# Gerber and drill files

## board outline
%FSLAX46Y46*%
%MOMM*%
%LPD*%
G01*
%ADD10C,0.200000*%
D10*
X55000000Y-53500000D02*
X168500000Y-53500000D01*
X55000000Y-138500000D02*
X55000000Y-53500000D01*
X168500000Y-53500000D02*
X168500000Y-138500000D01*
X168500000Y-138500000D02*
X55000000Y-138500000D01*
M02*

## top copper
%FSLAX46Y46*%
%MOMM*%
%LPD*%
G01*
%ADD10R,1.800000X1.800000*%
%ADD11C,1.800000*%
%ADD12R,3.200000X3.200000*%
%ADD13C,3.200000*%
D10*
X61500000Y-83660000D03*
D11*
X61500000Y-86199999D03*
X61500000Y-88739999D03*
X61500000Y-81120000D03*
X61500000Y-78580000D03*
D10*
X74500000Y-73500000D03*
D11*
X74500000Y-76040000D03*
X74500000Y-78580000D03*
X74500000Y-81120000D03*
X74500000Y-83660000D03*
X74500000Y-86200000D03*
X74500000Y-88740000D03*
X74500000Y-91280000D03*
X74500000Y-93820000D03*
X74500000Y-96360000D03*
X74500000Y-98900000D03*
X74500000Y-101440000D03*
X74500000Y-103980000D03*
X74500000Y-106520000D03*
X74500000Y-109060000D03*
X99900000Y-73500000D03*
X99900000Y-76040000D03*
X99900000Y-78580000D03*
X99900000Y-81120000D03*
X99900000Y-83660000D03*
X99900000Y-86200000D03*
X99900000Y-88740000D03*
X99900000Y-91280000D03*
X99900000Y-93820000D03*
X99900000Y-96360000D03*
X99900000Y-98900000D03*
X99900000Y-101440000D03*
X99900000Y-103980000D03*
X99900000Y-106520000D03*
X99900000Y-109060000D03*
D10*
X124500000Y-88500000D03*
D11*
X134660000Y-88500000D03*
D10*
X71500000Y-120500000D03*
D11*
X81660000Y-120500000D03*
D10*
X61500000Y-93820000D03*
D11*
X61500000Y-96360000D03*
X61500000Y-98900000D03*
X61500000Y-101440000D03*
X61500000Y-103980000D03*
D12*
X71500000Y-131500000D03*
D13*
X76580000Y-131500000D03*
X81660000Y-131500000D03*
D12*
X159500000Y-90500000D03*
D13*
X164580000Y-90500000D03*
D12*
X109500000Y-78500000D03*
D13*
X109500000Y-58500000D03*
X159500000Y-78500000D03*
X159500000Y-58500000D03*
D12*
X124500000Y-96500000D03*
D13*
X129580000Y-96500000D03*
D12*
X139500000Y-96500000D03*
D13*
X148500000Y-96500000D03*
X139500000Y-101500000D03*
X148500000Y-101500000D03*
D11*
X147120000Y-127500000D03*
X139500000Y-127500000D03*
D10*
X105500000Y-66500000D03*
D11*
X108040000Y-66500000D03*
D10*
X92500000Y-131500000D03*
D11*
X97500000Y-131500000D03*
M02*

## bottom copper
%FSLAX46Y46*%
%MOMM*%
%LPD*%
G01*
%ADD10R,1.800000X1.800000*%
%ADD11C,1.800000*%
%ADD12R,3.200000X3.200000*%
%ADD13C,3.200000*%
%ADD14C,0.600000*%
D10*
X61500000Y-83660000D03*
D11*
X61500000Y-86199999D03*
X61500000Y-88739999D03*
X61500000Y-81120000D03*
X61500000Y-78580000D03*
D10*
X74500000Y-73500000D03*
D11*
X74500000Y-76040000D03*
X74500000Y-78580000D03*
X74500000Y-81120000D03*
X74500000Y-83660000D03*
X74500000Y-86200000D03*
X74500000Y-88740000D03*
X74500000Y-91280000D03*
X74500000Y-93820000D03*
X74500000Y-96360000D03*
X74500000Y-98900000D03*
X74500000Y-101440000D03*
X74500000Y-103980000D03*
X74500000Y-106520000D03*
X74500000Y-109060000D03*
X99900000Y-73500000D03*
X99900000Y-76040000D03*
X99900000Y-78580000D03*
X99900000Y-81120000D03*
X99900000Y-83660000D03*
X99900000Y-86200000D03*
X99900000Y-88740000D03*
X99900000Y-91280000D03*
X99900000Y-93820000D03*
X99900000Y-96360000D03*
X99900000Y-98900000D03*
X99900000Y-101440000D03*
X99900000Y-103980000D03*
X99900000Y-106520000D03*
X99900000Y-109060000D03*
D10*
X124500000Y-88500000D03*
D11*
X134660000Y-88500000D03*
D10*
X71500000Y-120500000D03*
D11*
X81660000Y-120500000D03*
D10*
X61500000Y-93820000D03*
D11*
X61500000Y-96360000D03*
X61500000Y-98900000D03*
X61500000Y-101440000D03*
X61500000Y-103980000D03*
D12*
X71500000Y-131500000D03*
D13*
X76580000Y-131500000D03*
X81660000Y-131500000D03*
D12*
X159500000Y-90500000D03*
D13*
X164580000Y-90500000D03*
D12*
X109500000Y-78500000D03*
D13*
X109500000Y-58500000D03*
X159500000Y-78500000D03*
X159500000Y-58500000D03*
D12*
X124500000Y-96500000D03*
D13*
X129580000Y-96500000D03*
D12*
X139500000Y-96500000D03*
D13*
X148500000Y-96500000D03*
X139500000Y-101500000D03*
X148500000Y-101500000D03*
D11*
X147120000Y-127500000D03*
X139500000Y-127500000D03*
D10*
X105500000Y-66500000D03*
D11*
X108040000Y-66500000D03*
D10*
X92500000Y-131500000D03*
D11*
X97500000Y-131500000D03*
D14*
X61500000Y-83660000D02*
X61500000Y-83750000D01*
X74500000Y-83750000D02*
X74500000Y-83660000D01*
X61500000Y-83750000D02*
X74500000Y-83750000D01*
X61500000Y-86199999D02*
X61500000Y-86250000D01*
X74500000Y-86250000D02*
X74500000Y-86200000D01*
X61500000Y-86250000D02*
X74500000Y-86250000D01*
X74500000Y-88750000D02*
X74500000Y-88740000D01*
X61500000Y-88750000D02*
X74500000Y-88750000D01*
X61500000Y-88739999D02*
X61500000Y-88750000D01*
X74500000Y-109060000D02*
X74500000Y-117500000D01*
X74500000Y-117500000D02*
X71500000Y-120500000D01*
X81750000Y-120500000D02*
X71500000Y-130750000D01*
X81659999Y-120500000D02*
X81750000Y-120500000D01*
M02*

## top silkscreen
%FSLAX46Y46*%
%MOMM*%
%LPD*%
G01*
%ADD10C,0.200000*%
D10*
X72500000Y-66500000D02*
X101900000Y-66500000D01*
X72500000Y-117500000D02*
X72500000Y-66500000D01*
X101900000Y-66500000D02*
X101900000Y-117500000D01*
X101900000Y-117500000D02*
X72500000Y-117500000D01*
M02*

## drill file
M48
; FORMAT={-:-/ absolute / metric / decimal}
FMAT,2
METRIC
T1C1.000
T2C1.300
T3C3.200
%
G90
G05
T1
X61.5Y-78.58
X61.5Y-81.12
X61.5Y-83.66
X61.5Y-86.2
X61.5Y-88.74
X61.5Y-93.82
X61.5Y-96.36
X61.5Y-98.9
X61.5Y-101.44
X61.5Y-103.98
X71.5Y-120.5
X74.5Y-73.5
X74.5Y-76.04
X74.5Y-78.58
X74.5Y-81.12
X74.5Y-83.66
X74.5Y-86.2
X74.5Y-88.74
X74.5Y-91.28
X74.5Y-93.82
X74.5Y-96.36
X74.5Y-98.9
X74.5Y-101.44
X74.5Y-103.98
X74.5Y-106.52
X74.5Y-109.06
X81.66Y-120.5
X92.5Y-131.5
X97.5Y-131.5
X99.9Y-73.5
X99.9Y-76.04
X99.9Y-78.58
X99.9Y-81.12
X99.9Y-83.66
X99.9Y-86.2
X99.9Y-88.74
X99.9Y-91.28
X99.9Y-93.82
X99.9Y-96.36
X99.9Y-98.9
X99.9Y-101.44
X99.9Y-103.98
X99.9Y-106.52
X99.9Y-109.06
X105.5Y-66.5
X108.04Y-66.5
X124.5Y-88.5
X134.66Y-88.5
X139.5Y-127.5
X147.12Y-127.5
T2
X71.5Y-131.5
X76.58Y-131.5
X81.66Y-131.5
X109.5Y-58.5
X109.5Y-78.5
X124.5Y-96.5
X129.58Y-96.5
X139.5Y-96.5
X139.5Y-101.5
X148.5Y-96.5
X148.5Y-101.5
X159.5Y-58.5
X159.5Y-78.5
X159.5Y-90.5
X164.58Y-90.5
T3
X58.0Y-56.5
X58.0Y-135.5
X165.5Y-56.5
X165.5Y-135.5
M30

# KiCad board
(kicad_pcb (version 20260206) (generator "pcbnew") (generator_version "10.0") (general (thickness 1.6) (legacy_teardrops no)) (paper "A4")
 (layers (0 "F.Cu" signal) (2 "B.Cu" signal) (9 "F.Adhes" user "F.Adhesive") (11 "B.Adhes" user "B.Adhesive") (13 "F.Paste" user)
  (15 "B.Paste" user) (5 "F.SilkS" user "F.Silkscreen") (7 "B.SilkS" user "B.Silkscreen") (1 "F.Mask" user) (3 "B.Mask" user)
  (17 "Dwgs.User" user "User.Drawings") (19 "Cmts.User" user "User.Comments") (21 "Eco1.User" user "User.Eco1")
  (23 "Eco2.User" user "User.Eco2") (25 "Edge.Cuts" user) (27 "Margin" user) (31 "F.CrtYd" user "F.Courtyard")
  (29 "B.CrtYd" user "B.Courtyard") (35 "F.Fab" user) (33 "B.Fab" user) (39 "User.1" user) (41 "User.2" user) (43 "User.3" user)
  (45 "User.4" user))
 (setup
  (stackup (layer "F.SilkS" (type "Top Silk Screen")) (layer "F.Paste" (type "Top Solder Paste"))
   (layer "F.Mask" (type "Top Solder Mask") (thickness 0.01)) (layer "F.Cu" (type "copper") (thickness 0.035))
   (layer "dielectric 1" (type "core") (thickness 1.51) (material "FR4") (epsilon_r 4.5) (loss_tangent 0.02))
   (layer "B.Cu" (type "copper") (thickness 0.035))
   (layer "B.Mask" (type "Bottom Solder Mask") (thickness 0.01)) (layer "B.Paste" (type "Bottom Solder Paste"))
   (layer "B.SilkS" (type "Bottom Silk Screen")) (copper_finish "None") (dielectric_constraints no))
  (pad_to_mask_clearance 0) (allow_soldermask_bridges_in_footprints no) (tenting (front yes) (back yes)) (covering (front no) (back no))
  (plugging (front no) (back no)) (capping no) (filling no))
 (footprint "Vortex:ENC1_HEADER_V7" (layer "F.Cu") (at 61.5 83.5 -90)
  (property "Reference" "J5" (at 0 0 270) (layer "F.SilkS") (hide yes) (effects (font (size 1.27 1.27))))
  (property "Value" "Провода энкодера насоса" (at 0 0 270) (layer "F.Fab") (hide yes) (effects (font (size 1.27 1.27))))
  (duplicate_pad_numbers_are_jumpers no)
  (pad "1" thru_hole rect (at 0.16 0 270) (size 1.8 1.8) (drill 1) (layers "*.Cu") (remove_unused_layers no) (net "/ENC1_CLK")
   (thermal_bridge_angle 45))
  (pad "2" thru_hole circle (at 2.699999 0 270) (size 1.8 1.8) (drill 1) (layers "*.Cu") (remove_unused_layers no) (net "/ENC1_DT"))
  (pad "3" thru_hole circle (at 5.239999 0 270) (size 1.8 1.8) (drill 1) (layers "*.Cu") (remove_unused_layers no) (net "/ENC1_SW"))
  (pad "4" thru_hole circle (at -2.38 0 270) (size 1.8 1.8) (drill 1) (layers "*.Cu") (remove_unused_layers no) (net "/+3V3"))
  (pad "5" thru_hole circle (at -4.92 0 270) (size 1.8 1.8) (drill 1) (layers "*.Cu") (remove_unused_layers no) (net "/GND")))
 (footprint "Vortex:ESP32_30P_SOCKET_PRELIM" (layer "F.Cu") (at 74.5 73.5)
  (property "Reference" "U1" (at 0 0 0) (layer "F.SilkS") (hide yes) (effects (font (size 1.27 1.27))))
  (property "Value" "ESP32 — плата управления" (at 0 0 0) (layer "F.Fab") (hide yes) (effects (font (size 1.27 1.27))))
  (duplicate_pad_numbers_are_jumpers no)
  (fp_line (start -2 -7) (end 27.4 -7) (stroke (width 0.2) (type default)) (layer "F.SilkS"))
  (fp_line (start -2 44) (end -2 -7) (stroke (width 0.2) (type default)) (layer "F.SilkS"))
  (fp_line (start 27.4 -7) (end 27.4 44) (stroke (width 0.2) (type default)) (layer "F.SilkS"))
  (fp_line (start 27.4 44) (end -2 44) (stroke (width 0.2) (type default)) (layer "F.SilkS"))
  (pad "1" thru_hole rect (at 0 0) (size 1.8 1.8) (drill 1) (layers "*.Cu") (remove_unused_layers no) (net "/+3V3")
   (thermal_bridge_angle 45))
  (pad "2" thru_hole circle (at 0 2.54) (size 1.8 1.8) (drill 1) (layers "*.Cu") (remove_unused_layers no) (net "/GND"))
  (pad "3" thru_hole circle (at 0 5.08) (size 1.8 1.8) (drill 1) (layers "*.Cu") (remove_unused_layers no) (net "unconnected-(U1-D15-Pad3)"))
  (pad "4" thru_hole circle (at 0 7.62) (size 1.8 1.8) (drill 1) (layers "*.Cu") (remove_unused_layers no) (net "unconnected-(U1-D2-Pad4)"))
  (pad "5" thru_hole circle (at 0 10.16) (size 1.8 1.8) (drill 1) (layers "*.Cu") (remove_unused_layers no) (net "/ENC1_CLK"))
  (pad "6" thru_hole circle (at 0 12.7) (size 1.8 1.8) (drill 1) (layers "*.Cu") (remove_unused_layers no) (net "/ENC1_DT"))
  (pad "7" thru_hole circle (at 0 15.24) (size 1.8 1.8) (drill 1) (layers "*.Cu") (remove_unused_layers no) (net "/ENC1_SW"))
  (pad "8" thru_hole circle (at 0 17.78) (size 1.8 1.8) (drill 1) (layers "*.Cu") (remove_unused_layers no) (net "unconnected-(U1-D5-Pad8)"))
  (pad "9" thru_hole circle (at 0 20.32) (size 1.8 1.8) (drill 1) (layers "*.Cu") (remove_unused_layers no) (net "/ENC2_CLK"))
  (pad "10" thru_hole circle (at 0 22.86) (size 1.8 1.8) (drill 1) (layers "*.Cu") (remove_unused_layers no) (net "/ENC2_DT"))
  (pad "11" thru_hole circle (at 0 25.4) (size 1.8 1.8) (drill 1) (layers "*.Cu") (remove_unused_layers no) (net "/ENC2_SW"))
  (pad "12" thru_hole circle (at 0 27.94) (size 1.8 1.8) (drill 1) (layers "*.Cu") (remove_unused_layers no)
   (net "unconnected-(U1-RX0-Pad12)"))
  (pad "13" thru_hole circle (at 0 30.48) (size 1.8 1.8) (drill 1) (layers "*.Cu") (remove_unused_layers no)
   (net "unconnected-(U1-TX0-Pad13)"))
  (pad "14" thru_hole circle (at 0 33.02) (size 1.8 1.8) (drill 1) (layers "*.Cu") (remove_unused_layers no)
   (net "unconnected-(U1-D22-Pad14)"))
  (pad "15" thru_hole circle (at 0 35.56) (size 1.8 1.8) (drill 1) (layers "*.Cu") (remove_unused_layers no) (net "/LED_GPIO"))
  (pad "16" thru_hole circle (at 25.4 0) (size 1.8 1.8) (drill 1) (layers "*.Cu") (remove_unused_layers no) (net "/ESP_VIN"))
  (pad "17" thru_hole circle (at 25.4 2.54) (size 1.8 1.8) (drill 1) (layers "*.Cu") (remove_unused_layers no) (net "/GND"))
  (pad "18" thru_hole circle (at 25.4 5.08) (size 1.8 1.8) (drill 1) (layers "*.Cu") (remove_unused_layers no)
   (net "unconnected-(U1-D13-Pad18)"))
  (pad "19" thru_hole circle (at 25.4 7.62) (size 1.8 1.8) (drill 1) (layers "*.Cu") (remove_unused_layers no)
   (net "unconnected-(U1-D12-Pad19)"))
  (pad "20" thru_hole circle (at 25.4 10.16) (size 1.8 1.8) (drill 1) (layers "*.Cu") (remove_unused_layers no)
   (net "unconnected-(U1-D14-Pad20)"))
  (pad "21" thru_hole circle (at 25.4 12.7) (size 1.8 1.8) (drill 1) (layers "*.Cu") (remove_unused_layers no)
   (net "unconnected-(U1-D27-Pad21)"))
  (pad "22" thru_hole circle (at 25.4 15.24) (size 1.8 1.8) (drill 1) (layers "*.Cu") (remove_unused_layers no)
   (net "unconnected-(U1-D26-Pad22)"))
  (pad "23" thru_hole circle (at 25.4 17.78) (size 1.8 1.8) (drill 1) (layers "*.Cu") (remove_unused_layers no) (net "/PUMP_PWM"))
  (pad "24" thru_hole circle (at 25.4 20.32) (size 1.8 1.8) (drill 1) (layers "*.Cu") (remove_unused_layers no)
   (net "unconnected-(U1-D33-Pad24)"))
  (pad "25" thru_hole circle (at 25.4 22.86) (size 1.8 1.8) (drill 1) (layers "*.Cu") (remove_unused_layers no)
   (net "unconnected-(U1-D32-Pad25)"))
  (pad "26" thru_hole circle (at 25.4 25.4) (size 1.8 1.8) (drill 1) (layers "*.Cu") (remove_unused_layers no)
   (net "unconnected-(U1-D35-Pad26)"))
  (pad "27" thru_hole circle (at 25.4 27.94) (size 1.8 1.8) (drill 1) (layers "*.Cu") (remove_unused_layers no)
   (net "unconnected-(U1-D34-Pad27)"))
  (pad "28" thru_hole circle (at 25.4 30.48) (size 1.8 1.8) (drill 1) (layers "*.Cu") (remove_unused_layers no)
   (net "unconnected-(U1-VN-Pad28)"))
  (pad "29" thru_hole circle (at 25.4 33.02) (size 1.8 1.8) (drill 1) (layers "*.Cu") (remove_unused_layers no)
   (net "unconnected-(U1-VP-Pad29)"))
  (pad "30" thru_hole circle (at 25.4 35.56) (size 1.8 1.8) (drill 1) (layers "*.Cu") (remove_unused_layers no)
   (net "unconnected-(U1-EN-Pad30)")))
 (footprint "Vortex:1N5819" (layer "F.Cu") (at 124.5 88.5)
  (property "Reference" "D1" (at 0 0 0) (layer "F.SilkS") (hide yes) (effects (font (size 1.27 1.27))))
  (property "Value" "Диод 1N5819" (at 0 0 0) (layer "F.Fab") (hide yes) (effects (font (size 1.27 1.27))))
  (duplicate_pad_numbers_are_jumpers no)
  (pad "1" thru_hole rect (at 0 0) (size 1.8 1.8) (drill 1) (layers "*.Cu") (remove_unused_layers no) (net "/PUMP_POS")
   (thermal_bridge_angle 45))
  (pad "2" thru_hole circle (at 10.16 0) (size 1.8 1.8) (drill 1) (layers "*.Cu") (remove_unused_layers no) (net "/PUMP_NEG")))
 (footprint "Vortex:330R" (layer "F.Cu") (at 71.5 120.5)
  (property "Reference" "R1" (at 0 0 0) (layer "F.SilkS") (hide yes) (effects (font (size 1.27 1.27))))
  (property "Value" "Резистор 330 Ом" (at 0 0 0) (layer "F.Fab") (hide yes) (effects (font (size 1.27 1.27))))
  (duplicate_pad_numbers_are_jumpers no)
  (pad "1" thru_hole rect (at 0 0) (size 1.8 1.8) (drill 1) (layers "*.Cu") (remove_unused_layers no) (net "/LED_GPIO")
   (thermal_bridge_angle 45))
  (pad "2" thru_hole circle (at 10.16 0) (size 1.8 1.8) (drill 1) (layers "*.Cu") (remove_unused_layers no) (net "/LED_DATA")))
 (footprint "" (layer "F.Cu") (at 58 135.5)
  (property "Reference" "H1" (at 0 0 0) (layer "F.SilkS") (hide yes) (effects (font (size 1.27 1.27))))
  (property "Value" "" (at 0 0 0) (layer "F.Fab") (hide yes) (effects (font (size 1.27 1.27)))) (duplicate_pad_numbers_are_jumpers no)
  (pad "" np_thru_hole circle (at 0 0) (size 3.2 3.2) (drill 3.2) (layers "*.Cu")))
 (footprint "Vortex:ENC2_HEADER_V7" (layer "F.Cu") (at 61.5 96.5 -90)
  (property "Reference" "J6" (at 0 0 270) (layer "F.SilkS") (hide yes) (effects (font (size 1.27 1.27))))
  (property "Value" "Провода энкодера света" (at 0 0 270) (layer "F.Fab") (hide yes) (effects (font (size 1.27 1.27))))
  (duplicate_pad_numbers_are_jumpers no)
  (pad "1" thru_hole rect (at -2.68 0 270) (size 1.8 1.8) (drill 1) (layers "*.Cu") (remove_unused_layers no) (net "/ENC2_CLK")
   (thermal_bridge_angle 45))
  (pad "2" thru_hole circle (at -0.14 0 270) (size 1.8 1.8) (drill 1) (layers "*.Cu") (remove_unused_layers no) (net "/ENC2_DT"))
  (pad "3" thru_hole circle (at 2.4 0 270) (size 1.8 1.8) (drill 1) (layers "*.Cu") (remove_unused_layers no) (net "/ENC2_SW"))
  (pad "4" thru_hole circle (at 4.94 0 270) (size 1.8 1.8) (drill 1) (layers "*.Cu") (remove_unused_layers no) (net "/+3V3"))
  (pad "5" thru_hole circle (at 7.48 0 270) (size 1.8 1.8) (drill 1) (layers "*.Cu") (remove_unused_layers no) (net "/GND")))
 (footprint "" (layer "F.Cu") (at 58 56.5)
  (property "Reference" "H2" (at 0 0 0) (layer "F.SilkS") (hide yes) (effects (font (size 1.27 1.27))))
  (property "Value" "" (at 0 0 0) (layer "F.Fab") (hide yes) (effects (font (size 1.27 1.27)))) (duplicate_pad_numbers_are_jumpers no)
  (pad "" np_thru_hole circle (at 0 0) (size 3.2 3.2) (drill 3.2) (layers "*.Cu")))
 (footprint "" (layer "F.Cu") (at 165.5 135.5)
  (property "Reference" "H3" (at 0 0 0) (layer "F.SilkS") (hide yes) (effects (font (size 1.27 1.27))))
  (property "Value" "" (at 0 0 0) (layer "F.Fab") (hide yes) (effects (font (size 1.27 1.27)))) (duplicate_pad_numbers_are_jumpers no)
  (pad "" np_thru_hole circle (at 0 0) (size 3.2 3.2) (drill 3.2) (layers "*.Cu")))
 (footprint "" (layer "F.Cu") (at 165.5 56.5)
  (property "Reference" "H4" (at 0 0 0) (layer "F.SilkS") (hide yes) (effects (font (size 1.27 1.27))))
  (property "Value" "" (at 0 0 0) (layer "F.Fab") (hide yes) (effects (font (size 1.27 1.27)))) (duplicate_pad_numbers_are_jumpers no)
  (pad "" np_thru_hole circle (at 0 0) (size 3.2 3.2) (drill 3.2) (layers "*.Cu")))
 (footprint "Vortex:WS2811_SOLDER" (layer "F.Cu") (at 71.5 131.5)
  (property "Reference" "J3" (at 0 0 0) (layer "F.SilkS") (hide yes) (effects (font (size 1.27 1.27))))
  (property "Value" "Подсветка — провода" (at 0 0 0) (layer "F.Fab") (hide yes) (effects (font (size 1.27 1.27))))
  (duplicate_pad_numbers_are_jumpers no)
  (pad "1" thru_hole rect (at 0 0) (size 3.2 3.2) (drill 1.3) (layers "*.Cu") (remove_unused_layers no) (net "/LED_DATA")
   (thermal_bridge_angle 45))
  (pad "2" thru_hole circle (at 5.08 0) (size 3.2 3.2) (drill 1.3) (layers "*.Cu") (remove_unused_layers no) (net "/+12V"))
  (pad "3" thru_hole circle (at 10.16 0) (size 3.2 3.2) (drill 1.3) (layers "*.Cu") (remove_unused_layers no) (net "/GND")))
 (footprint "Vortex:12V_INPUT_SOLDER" (layer "F.Cu") (at 159.5 90.5)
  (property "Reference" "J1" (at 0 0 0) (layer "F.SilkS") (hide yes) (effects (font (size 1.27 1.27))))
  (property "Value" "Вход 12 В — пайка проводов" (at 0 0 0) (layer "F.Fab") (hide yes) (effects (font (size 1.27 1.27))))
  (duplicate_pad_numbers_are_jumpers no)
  (pad "1" thru_hole rect (at 0 0) (size 3.2 3.2) (drill 1.3) (layers "*.Cu") (remove_unused_layers no) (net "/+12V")
   (thermal_bridge_angle 45))
  (pad "2" thru_hole circle (at 5.08 0) (size 3.2 3.2) (drill 1.3) (layers "*.Cu") (remove_unused_layers no) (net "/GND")))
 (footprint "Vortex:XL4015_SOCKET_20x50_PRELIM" (layer "F.Cu") (at 109.5 78.5 90)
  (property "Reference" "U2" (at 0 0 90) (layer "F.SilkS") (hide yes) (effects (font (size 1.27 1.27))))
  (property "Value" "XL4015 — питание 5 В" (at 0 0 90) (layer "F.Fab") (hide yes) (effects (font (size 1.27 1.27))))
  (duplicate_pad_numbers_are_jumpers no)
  (pad "1" thru_hole rect (at 0 0 90) (size 3.2 3.2) (drill 1.3) (layers "*.Cu") (remove_unused_layers no) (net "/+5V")
   (thermal_bridge_angle 45))
  (pad "2" thru_hole circle (at 20 0 90) (size 3.2 3.2) (drill 1.3) (layers "*.Cu") (remove_unused_layers no) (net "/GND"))
  (pad "3" thru_hole circle (at 0 50 90) (size 3.2 3.2) (drill 1.3) (layers "*.Cu") (remove_unused_layers no) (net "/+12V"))
  (pad "4" thru_hole circle (at 20 50 90) (size 3.2 3.2) (drill 1.3) (layers "*.Cu") (remove_unused_layers no) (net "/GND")))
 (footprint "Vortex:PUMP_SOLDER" (layer "F.Cu") (at 124.5 96.5)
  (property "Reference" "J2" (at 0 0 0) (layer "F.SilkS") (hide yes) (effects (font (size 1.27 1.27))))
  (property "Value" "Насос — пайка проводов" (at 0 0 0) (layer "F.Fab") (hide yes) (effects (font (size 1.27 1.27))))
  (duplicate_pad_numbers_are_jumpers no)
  (pad "1" thru_hole rect (at 0 0) (size 3.2 3.2) (drill 1.3) (layers "*.Cu") (remove_unused_layers no) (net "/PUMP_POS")
   (thermal_bridge_angle 45))
  (pad "2" thru_hole circle (at 5.08 0) (size 3.2 3.2) (drill 1.3) (layers "*.Cu") (remove_unused_layers no) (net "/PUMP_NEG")))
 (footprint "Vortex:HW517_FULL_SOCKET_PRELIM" (layer "F.Cu") (at 139.5 96.5)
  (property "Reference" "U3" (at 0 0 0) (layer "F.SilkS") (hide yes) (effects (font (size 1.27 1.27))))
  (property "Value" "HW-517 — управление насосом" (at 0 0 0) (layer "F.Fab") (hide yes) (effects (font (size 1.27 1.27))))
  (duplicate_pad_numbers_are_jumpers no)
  (pad "1" thru_hole rect (at 0 0) (size 3.2 3.2) (drill 1.3) (layers "*.Cu") (remove_unused_layers no) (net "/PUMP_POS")
   (thermal_bridge_angle 45))
  (pad "2" thru_hole circle (at 9 0) (size 3.2 3.2) (drill 1.3) (layers "*.Cu") (remove_unused_layers no) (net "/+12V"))
  (pad "3" thru_hole circle (at 0 5) (size 3.2 3.2) (drill 1.3) (layers "*.Cu") (remove_unused_layers no) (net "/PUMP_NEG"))
  (pad "4" thru_hole circle (at 9 5) (size 3.2 3.2) (drill 1.3) (layers "*.Cu") (remove_unused_layers no) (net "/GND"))
  (pad "5" thru_hole circle (at 7.62 31) (size 1.8 1.8) (drill 1) (layers "*.Cu") (remove_unused_layers no) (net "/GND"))
  (pad "6" thru_hole circle (at 0 31) (size 1.8 1.8) (drill 1) (layers "*.Cu") (remove_unused_layers no) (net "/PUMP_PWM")))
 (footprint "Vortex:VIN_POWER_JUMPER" (layer "F.Cu") (at 105.5 66.5)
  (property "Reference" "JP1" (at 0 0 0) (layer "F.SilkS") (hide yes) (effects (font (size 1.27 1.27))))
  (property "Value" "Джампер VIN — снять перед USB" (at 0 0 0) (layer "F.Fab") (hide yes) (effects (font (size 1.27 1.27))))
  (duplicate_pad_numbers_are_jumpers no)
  (pad "1" thru_hole rect (at 0 0) (size 1.8 1.8) (drill 1) (layers "*.Cu") (remove_unused_layers no) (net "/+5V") (thermal_bridge_angle 45))
  (pad "2" thru_hole circle (at 2.54 0) (size 1.8 1.8) (drill 1) (layers "*.Cu") (remove_unused_layers no) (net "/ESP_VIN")))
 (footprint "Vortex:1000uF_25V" (layer "F.Cu") (at 92.5 131.5)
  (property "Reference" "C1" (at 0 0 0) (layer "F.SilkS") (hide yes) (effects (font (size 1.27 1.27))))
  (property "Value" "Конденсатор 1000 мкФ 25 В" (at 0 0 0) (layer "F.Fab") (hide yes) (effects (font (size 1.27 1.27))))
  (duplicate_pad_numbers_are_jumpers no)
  (pad "1" thru_hole rect (at 0 0) (size 1.8 1.8) (drill 1) (layers "*.Cu") (remove_unused_layers no) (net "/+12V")
   (thermal_bridge_angle 45))
  (pad "2" thru_hole circle (at 5 0) (size 1.8 1.8) (drill 1) (layers "*.Cu") (remove_unused_layers no) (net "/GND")))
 (gr_line (start 55 53.5) (end 168.5 53.5) (stroke (width 0.2) (type default)) (layer "Edge.Cuts"))
 (gr_line (start 55 138.5) (end 55 53.5) (stroke (width 0.2) (type default)) (layer "Edge.Cuts"))
 (gr_line (start 168.5 53.5) (end 168.5 138.5) (stroke (width 0.2) (type default)) (layer "Edge.Cuts"))
 (gr_line (start 168.5 138.5) (end 55 138.5) (stroke (width 0.2) (type default)) (layer "Edge.Cuts"))
 (segment (start 61.5 83.66) (end 61.5 83.75) (width 0.6) (layer "B.Cu") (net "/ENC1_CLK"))
 (segment (start 74.5 83.75) (end 74.5 83.66) (width 0.6) (layer "B.Cu") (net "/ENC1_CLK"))
 (segment (start 61.5 83.75) (end 74.5 83.75) (width 0.6) (layer "B.Cu") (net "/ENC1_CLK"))
 (segment (start 61.5 86.199999) (end 61.5 86.25) (width 0.6) (layer "B.Cu") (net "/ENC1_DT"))
 (segment (start 74.5 86.25) (end 74.5 86.2) (width 0.6) (layer "B.Cu") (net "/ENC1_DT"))
 (segment (start 61.5 86.25) (end 74.5 86.25) (width 0.6) (layer "B.Cu") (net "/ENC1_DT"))
 (segment (start 74.5 88.75) (end 74.5 88.74) (width 0.6) (layer "B.Cu") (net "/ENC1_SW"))
 (segment (start 61.5 88.75) (end 74.5 88.75) (width 0.6) (layer "B.Cu") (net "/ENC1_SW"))
 (segment (start 61.5 88.739999) (end 61.5 88.75) (width 0.6) (layer "B.Cu") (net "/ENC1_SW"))
 (segment (start 74.5 109.06) (end 74.5 117.5) (width 0.6) (layer "B.Cu") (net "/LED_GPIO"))
 (segment (start 74.5 117.5) (end 71.5 120.5) (width 0.6) (layer "B.Cu") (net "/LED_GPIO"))
 (segment (start 81.75 120.5) (end 71.5 130.75) (width 0.6) (layer "B.Cu") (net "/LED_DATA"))
 (segment (start 81.659999 120.5) (end 81.75 120.5) (width 0.6) (layer "B.Cu") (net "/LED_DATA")))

